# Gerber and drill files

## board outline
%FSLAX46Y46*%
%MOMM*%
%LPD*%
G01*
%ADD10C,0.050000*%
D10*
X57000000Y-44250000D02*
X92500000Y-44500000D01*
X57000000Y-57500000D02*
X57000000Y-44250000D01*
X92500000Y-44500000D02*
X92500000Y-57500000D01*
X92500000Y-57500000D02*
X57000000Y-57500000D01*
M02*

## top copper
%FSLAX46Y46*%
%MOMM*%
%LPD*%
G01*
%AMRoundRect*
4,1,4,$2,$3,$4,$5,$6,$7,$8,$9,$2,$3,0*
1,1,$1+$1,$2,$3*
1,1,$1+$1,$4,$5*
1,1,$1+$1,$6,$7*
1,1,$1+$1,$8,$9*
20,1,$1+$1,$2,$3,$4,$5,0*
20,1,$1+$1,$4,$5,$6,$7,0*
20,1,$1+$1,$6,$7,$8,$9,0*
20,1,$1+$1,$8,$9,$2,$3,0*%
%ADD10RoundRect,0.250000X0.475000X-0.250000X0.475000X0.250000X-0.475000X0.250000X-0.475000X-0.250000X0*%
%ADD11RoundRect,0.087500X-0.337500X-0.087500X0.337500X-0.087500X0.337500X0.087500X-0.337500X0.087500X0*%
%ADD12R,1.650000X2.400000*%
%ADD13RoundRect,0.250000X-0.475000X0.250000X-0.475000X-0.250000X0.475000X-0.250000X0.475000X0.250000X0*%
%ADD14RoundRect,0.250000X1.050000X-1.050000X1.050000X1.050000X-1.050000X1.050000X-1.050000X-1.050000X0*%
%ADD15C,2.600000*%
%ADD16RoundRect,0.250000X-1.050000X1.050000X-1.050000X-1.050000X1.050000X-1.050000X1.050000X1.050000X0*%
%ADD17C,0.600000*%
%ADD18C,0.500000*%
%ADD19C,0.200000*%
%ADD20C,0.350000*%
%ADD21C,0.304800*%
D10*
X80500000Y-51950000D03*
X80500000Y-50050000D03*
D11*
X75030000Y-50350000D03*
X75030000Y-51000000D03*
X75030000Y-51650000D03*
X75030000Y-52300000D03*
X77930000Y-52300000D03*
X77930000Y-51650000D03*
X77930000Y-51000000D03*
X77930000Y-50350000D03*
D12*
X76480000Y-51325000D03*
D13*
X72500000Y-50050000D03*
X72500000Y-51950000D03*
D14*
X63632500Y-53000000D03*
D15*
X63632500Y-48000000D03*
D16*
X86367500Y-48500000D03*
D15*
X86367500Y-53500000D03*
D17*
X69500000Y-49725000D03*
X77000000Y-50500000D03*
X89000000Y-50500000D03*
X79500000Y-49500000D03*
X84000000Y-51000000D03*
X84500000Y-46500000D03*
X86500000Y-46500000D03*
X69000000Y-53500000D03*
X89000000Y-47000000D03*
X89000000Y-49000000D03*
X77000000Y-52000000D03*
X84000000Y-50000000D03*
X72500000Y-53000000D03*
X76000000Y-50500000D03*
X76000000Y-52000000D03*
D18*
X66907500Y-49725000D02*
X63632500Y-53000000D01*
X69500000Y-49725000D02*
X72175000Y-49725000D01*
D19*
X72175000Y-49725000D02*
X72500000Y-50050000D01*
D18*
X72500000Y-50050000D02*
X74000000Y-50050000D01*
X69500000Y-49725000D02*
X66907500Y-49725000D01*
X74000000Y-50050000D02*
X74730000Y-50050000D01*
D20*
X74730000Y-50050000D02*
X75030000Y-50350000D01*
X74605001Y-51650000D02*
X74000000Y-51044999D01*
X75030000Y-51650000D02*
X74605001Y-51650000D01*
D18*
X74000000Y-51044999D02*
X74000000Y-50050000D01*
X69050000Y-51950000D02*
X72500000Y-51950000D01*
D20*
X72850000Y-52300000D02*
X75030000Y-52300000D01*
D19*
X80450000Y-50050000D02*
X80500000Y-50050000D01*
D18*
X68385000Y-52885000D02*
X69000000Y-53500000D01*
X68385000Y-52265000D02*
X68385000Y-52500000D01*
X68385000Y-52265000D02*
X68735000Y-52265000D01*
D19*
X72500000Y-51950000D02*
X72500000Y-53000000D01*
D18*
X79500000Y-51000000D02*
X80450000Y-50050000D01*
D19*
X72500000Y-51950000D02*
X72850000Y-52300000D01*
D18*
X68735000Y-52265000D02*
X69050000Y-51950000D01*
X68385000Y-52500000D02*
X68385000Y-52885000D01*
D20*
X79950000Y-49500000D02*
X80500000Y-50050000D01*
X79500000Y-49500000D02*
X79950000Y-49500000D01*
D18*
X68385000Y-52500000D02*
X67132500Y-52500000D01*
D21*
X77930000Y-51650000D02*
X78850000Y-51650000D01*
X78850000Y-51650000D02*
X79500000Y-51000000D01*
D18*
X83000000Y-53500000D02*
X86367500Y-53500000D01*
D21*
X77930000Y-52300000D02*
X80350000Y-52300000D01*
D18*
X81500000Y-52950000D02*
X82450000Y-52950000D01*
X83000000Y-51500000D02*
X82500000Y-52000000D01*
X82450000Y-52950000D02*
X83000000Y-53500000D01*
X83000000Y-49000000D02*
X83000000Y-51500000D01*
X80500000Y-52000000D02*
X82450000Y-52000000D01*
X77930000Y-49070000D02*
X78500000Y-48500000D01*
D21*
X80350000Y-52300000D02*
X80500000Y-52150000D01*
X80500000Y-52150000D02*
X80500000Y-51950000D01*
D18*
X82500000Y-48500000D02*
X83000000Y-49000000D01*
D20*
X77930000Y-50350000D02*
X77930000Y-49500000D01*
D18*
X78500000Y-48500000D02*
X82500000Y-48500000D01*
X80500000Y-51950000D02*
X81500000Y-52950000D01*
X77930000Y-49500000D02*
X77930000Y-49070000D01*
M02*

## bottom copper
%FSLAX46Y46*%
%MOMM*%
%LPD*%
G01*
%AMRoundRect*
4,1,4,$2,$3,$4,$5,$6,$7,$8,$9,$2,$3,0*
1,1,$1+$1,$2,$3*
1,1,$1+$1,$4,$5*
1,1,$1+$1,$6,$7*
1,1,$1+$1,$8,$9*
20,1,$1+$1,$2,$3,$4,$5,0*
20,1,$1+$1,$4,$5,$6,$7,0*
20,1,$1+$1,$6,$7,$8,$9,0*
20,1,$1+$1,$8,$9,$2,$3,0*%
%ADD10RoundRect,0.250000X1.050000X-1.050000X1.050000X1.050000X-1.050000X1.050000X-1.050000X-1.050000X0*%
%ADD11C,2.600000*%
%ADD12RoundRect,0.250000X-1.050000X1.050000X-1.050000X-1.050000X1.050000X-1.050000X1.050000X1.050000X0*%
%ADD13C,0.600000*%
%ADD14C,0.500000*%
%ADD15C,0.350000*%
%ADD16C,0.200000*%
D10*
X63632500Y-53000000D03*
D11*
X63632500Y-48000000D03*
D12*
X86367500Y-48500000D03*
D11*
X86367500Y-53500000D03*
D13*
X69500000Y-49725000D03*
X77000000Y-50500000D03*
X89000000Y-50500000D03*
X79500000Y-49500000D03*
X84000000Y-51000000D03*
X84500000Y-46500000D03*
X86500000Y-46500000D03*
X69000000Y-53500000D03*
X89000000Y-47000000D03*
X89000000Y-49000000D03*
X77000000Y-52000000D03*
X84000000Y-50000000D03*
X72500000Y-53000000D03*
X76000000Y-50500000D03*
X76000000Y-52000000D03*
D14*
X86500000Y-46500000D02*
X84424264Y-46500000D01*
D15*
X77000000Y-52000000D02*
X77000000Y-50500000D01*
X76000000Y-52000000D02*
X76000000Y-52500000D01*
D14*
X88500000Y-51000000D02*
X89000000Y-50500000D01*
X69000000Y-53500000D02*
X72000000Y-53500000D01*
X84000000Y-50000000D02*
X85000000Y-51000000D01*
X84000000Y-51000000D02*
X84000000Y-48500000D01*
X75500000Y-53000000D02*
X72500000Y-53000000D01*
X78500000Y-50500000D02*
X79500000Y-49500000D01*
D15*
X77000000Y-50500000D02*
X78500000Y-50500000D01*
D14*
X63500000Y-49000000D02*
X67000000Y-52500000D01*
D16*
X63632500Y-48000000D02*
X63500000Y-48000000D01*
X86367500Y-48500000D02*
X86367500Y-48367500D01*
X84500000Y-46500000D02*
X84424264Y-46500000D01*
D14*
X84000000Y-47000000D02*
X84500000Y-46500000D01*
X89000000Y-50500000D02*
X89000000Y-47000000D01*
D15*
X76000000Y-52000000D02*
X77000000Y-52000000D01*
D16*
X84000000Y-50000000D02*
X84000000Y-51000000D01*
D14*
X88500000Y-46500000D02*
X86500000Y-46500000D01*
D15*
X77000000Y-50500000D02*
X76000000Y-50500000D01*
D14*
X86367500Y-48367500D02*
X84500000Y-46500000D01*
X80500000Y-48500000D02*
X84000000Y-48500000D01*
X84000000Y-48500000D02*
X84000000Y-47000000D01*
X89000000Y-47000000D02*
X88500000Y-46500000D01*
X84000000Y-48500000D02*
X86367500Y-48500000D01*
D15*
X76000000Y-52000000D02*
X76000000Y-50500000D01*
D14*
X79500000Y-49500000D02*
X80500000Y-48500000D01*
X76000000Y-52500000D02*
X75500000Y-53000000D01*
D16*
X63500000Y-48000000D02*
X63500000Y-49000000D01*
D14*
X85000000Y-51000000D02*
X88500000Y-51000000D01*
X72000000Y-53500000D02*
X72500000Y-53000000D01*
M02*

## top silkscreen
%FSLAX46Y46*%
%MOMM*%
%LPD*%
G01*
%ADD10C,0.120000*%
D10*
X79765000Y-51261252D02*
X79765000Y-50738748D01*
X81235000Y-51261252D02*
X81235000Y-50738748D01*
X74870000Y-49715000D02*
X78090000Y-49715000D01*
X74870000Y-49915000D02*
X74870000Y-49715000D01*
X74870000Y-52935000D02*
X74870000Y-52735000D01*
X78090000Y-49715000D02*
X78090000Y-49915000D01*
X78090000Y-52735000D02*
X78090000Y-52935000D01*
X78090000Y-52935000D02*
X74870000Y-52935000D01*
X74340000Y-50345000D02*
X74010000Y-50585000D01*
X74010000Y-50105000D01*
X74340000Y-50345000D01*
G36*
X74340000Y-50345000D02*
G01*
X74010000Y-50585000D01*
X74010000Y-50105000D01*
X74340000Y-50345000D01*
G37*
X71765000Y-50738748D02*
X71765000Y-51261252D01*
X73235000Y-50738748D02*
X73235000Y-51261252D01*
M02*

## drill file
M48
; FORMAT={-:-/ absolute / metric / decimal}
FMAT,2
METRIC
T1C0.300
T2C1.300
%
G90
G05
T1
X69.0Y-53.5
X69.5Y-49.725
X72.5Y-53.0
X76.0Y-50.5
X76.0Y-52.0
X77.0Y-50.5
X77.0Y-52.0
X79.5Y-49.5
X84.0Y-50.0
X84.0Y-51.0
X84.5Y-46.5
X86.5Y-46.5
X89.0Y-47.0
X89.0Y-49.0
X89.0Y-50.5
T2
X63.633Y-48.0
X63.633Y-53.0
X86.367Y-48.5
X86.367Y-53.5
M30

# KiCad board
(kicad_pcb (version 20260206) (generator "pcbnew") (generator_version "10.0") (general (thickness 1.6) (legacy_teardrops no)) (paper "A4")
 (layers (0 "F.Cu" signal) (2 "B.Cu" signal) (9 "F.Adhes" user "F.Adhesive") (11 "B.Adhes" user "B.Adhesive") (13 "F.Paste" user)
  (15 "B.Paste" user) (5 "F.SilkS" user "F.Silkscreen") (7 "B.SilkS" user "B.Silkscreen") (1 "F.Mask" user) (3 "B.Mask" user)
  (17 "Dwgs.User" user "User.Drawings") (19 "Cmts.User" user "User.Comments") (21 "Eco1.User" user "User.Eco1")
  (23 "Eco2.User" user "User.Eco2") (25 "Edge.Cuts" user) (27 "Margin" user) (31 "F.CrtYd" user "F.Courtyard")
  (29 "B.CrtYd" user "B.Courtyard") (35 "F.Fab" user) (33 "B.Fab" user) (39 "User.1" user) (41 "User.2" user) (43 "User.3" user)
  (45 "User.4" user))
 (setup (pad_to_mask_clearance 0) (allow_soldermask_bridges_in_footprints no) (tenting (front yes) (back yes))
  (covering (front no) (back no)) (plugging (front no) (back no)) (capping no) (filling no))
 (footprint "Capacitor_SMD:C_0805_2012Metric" (layer "F.Cu") (at 80.5 51 90)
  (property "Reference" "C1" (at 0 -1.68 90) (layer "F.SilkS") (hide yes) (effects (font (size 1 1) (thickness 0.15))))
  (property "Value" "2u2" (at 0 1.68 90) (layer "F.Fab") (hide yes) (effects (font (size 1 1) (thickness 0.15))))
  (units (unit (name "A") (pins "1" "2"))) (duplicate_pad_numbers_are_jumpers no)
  (fp_line (start -0.261252 -0.735) (end 0.261252 -0.735) (stroke (width 0.12) (type solid)) (layer "F.SilkS"))
  (fp_line (start -0.261252 0.735) (end 0.261252 0.735) (stroke (width 0.12) (type solid)) (layer "F.SilkS"))
  (pad "1" smd roundrect (at -0.95 0 90) (size 1 1.45) (layers "F.Cu" "F.Mask" "F.Paste") (roundrect_rratio 0.25) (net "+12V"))
  (pad "2" smd roundrect (at 0.95 0 90) (size 1 1.45) (layers "F.Cu" "F.Mask" "F.Paste") (roundrect_rratio 0.25) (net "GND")))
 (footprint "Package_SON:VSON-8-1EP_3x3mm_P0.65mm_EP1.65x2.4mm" (layer "F.Cu") (at 76.48 51.325)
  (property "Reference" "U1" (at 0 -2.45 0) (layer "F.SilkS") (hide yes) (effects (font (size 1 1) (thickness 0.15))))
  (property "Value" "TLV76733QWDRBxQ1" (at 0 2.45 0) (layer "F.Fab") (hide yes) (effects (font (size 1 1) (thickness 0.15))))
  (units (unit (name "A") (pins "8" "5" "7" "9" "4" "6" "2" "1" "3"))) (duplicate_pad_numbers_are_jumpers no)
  (fp_line (start -1.61 -1.61) (end 1.61 -1.61) (stroke (width 0.12) (type solid)) (layer "F.SilkS"))
  (fp_line (start -1.61 -1.41) (end -1.61 -1.61) (stroke (width 0.12) (type solid)) (layer "F.SilkS"))
  (fp_line (start -1.61 1.61) (end -1.61 1.41) (stroke (width 0.12) (type solid)) (layer "F.SilkS"))
  (fp_line (start 1.61 -1.61) (end 1.61 -1.41) (stroke (width 0.12) (type solid)) (layer "F.SilkS"))
  (fp_line (start 1.61 1.41) (end 1.61 1.61) (stroke (width 0.12) (type solid)) (layer "F.SilkS"))
  (fp_line (start 1.61 1.61) (end -1.61 1.61) (stroke (width 0.12) (type solid)) (layer "F.SilkS"))
  (fp_poly (pts (xy -2.14 -0.98) (xy -2.47 -0.74) (xy -2.47 -1.22)) (stroke (width 0.12) (type solid)) (fill yes) (layer "F.SilkS"))
  (pad "" smd roundrect (at 0 -0.6) (size 1.33 0.97) (layers "F.Paste") (roundrect_rratio 0.25))
  (pad "" smd roundrect (at 0 0.6) (size 1.33 0.97) (layers "F.Paste") (roundrect_rratio 0.25))
  (pad "1" smd roundrect (at -1.45 -0.975) (size 0.85 0.35) (layers "F.Cu" "F.Mask" "F.Paste") (roundrect_rratio 0.25) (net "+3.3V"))
  (pad "2" smd roundrect (at -1.45 -0.325) (size 0.85 0.35) (layers "F.Cu" "F.Mask" "F.Paste") (roundrect_rratio 0.25)
   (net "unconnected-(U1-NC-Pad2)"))
  (pad "3" smd roundrect (at -1.45 0.325) (size 0.85 0.35) (layers "F.Cu" "F.Mask" "F.Paste") (roundrect_rratio 0.25) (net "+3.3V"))
  (pad "4" smd roundrect (at -1.45 0.975) (size 0.85 0.35) (layers "F.Cu" "F.Mask" "F.Paste") (roundrect_rratio 0.25) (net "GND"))
  (pad "5" smd roundrect (at 1.45 0.975) (size 0.85 0.35) (layers "F.Cu" "F.Mask" "F.Paste") (roundrect_rratio 0.25) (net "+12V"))
  (pad "6" smd roundrect (at 1.45 0.325) (size 0.85 0.35) (layers "F.Cu" "F.Mask" "F.Paste") (roundrect_rratio 0.25) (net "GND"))
  (pad "7" smd roundrect (at 1.45 -0.325) (size 0.85 0.35) (layers "F.Cu" "F.Mask" "F.Paste") (roundrect_rratio 0.25)
   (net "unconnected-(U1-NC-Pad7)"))
  (pad "8" smd roundrect (at 1.45 -0.975) (size 0.85 0.35) (layers "F.Cu" "F.Mask" "F.Paste") (roundrect_rratio 0.25) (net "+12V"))
  (pad "9" smd rect (at 0 0) (size 1.65 2.4) (layers "F.Cu" "F.Mask") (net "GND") (zone_connect 2)))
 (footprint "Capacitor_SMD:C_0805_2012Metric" (layer "F.Cu") (at 72.5 51 -90)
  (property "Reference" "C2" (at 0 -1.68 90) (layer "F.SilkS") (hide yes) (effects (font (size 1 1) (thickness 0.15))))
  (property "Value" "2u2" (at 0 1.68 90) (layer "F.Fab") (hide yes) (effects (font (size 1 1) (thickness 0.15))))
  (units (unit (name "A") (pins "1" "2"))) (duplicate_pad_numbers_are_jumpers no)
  (fp_line (start -0.261252 0.735) (end 0.261252 0.735) (stroke (width 0.12) (type solid)) (layer "F.SilkS"))
  (fp_line (start -0.261252 -0.735) (end 0.261252 -0.735) (stroke (width 0.12) (type solid)) (layer "F.SilkS"))
  (pad "1" smd roundrect (at -0.95 0 270) (size 1 1.45) (layers "F.Cu" "F.Mask" "F.Paste") (roundrect_rratio 0.25) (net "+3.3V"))
  (pad "2" smd roundrect (at 0.95 0 270) (size 1 1.45) (layers "F.Cu" "F.Mask" "F.Paste") (roundrect_rratio 0.25) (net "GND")))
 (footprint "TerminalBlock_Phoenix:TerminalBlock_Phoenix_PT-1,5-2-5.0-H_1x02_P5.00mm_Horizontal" (layer "B.Cu") (at 63.6325 53 90)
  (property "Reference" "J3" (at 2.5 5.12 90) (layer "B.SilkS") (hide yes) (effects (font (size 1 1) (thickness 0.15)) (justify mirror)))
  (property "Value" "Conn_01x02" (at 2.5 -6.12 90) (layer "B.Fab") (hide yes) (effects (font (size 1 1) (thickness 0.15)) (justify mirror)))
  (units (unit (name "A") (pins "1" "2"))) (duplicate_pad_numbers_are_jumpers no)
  (pad "1" thru_hole roundrect (at 0 0 90) (size 2.6 2.6) (drill 1.3) (layers "*.Cu" "*.Mask") (remove_unused_layers no)
   (roundrect_rratio 0.096154) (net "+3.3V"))
  (pad "2" thru_hole circle (at 5 0 90) (size 2.6 2.6) (drill 1.3) (layers "*.Cu" "*.Mask") (remove_unused_layers no) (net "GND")))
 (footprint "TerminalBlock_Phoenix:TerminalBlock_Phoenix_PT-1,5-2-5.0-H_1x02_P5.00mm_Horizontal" (layer "B.Cu") (at 86.3675 48.5 -90)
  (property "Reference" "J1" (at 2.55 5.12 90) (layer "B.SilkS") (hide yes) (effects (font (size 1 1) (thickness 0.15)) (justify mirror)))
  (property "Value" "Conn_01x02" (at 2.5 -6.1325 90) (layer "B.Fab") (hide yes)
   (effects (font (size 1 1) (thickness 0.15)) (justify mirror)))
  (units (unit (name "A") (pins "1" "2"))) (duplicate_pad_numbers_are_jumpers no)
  (pad "1" thru_hole roundrect (at 0 0 270) (size 2.6 2.6) (drill 1.3) (layers "*.Cu" "*.Mask") (remove_unused_layers no)
   (roundrect_rratio 0.096154) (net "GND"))
  (pad "2" thru_hole circle (at 5 0 270) (size 2.6 2.6) (drill 1.3) (layers "*.Cu" "*.Mask") (remove_unused_layers no) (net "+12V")))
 (gr_line (start 57 44.25) (end 92.5 44.5) (stroke (width 0.05) (type default)) (layer "Edge.Cuts"))
 (gr_line (start 57 57.5) (end 57 44.25) (stroke (width 0.05) (type default)) (layer "Edge.Cuts"))
 (gr_line (start 92.5 44.5) (end 92.5 57.5) (stroke (width 0.05) (type default)) (layer "Edge.Cuts"))
 (gr_line (start 92.5 57.5) (end 57 57.5) (stroke (width 0.05) (type solid)) (layer "Edge.Cuts"))
 (segment (start 66.9075 49.725) (end 63.6325 53) (width 0.5) (layer "F.Cu") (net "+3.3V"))
 (segment (start 69.5 49.725) (end 72.175 49.725) (width 0.5) (layer "F.Cu") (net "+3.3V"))
 (segment (start 72.175 49.725) (end 72.5 50.05) (width 0.2) (layer "F.Cu") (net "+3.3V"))
 (segment (start 72.5 50.05) (end 74 50.05) (width 0.5) (layer "F.Cu") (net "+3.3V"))
 (segment (start 69.5 49.725) (end 66.9075 49.725) (width 0.5) (layer "F.Cu") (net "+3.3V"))
 (segment (start 74 50.05) (end 74.73 50.05) (width 0.5) (layer "F.Cu") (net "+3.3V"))
 (segment (start 74.73 50.05) (end 75.03 50.35) (width 0.35) (layer "F.Cu") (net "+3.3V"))
 (segment (start 74.605001 51.65) (end 74 51.044999) (width 0.35) (layer "F.Cu") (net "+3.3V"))
 (segment (start 75.03 51.65) (end 74.605001 51.65) (width 0.35) (layer "F.Cu") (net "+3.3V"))
 (segment (start 74 51.044999) (end 74 50.05) (width 0.5) (layer "F.Cu") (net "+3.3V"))
 (via (at 69.5 49.725) (size 0.6) (drill 0.3) (layers "F.Cu" "B.Cu") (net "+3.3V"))
 (segment (start 69.05 51.95) (end 72.5 51.95) (width 0.5) (layer "F.Cu") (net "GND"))
 (segment (start 72.85 52.3) (end 75.03 52.3) (width 0.35) (layer "F.Cu") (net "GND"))
 (segment (start 80.45 50.05) (end 80.5 50.05) (width 0.2) (layer "F.Cu") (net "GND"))
 (segment (start 68.385 52.885) (end 69 53.5) (width 0.5) (layer "F.Cu") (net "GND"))
 (segment (start 68.385 52.265) (end 68.385 52.5) (width 0.5) (layer "F.Cu") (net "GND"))
 (segment (start 68.385 52.265) (end 68.735 52.265) (width 0.5) (layer "F.Cu") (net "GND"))
 (segment (start 72.5 51.95) (end 72.5 53) (width 0.2) (layer "F.Cu") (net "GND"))
 (segment (start 79.5 51) (end 80.45 50.05) (width 0.5) (layer "F.Cu") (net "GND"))
 (segment (start 72.5 51.95) (end 72.85 52.3) (width 0.2) (layer "F.Cu") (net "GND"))
 (segment (start 68.735 52.265) (end 69.05 51.95) (width 0.5) (layer "F.Cu") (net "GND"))
 (segment (start 68.385 52.5) (end 68.385 52.885) (width 0.5) (layer "F.Cu") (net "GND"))
 (segment (start 79.95 49.5) (end 80.5 50.05) (width 0.35) (layer "F.Cu") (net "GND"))
 (segment (start 79.5 49.5) (end 79.95 49.5) (width 0.35) (layer "F.Cu") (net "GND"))
 (segment (start 68.385 52.5) (end 67.1325 52.5) (width 0.5) (layer "F.Cu") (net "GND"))
 (segment (start 77.93 51.65) (end 78.85 51.65) (width 0.3048) (layer "F.Cu") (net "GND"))
 (segment (start 78.85 51.65) (end 79.5 51) (width 0.3048) (layer "F.Cu") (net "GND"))
 (via (at 77 50.5) (size 0.6) (drill 0.3) (layers "F.Cu" "B.Cu") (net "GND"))
 (via (at 89 50.5) (size 0.6) (drill 0.3) (layers "F.Cu" "B.Cu") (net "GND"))
 (via (at 79.5 49.5) (size 0.6) (drill 0.3) (layers "F.Cu" "B.Cu") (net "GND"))
 (via (at 84 51) (size 0.6) (drill 0.3) (layers "F.Cu" "B.Cu") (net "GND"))
 (via (at 84.5 46.5) (size 0.6) (drill 0.3) (layers "F.Cu" "B.Cu") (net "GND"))
 (via (at 86.5 46.5) (size 0.6) (drill 0.3) (layers "F.Cu" "B.Cu") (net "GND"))
 (via (at 69 53.5) (size 0.6) (drill 0.3) (layers "F.Cu" "B.Cu") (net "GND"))
 (via (at 89 47) (size 0.6) (drill 0.3) (layers "F.Cu" "B.Cu") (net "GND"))
 (via (at 89 49) (size 0.6) (drill 0.3) (layers "F.Cu" "B.Cu") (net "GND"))
 (via (at 77 52) (size 0.6) (drill 0.3) (layers "F.Cu" "B.Cu") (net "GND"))
 (via (at 84 50) (size 0.6) (drill 0.3) (layers "F.Cu" "B.Cu") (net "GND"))
 (via (at 72.5 53) (size 0.6) (drill 0.3) (layers "F.Cu" "B.Cu") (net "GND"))
 (via (at 76 50.5) (size 0.6) (drill 0.3) (layers "F.Cu" "B.Cu") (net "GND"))
 (via (at 76 52) (size 0.6) (drill 0.3) (layers "F.Cu" "B.Cu") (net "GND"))
 (segment (start 86.5 46.5) (end 84.424264 46.5) (width 0.5) (layer "B.Cu") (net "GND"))
 (segment (start 77 52) (end 77 50.5) (width 0.35) (layer "B.Cu") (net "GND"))
 (segment (start 76 52) (end 76 52.5) (width 0.35) (layer "B.Cu") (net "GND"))
 (segment (start 88.5 51) (end 89 50.5) (width 0.5) (layer "B.Cu") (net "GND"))
 (segment (start 69 53.5) (end 72 53.5) (width 0.5) (layer "B.Cu") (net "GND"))
 (segment (start 84 50) (end 85 51) (width 0.5) (layer "B.Cu") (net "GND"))
 (segment (start 84 51) (end 84 48.5) (width 0.5) (layer "B.Cu") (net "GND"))
 (segment (start 75.5 53) (end 72.5 53) (width 0.5) (layer "B.Cu") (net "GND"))
 (segment (start 78.5 50.5) (end 79.5 49.5) (width 0.5) (layer "B.Cu") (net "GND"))
 (segment (start 77 50.5) (end 78.5 50.5) (width 0.35) (layer "B.Cu") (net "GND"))
 (segment (start 63.5 49) (end 67 52.5) (width 0.5) (layer "B.Cu") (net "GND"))
 (segment (start 63.6325 48) (end 63.5 48) (width 0.2) (layer "B.Cu") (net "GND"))
 (segment (start 86.3675 48.5) (end 86.3675 48.3675) (width 0.2) (layer "B.Cu") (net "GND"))
 (segment (start 84.5 46.5) (end 84.424264 46.5) (width 0.2) (layer "B.Cu") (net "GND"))
 (segment (start 84 47) (end 84.5 46.5) (width 0.5) (layer "B.Cu") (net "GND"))
 (segment (start 89 50.5) (end 89 47) (width 0.5) (layer "B.Cu") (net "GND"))
 (segment (start 76 52) (end 77 52) (width 0.35) (layer "B.Cu") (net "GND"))
 (segment (start 84 50) (end 84 51) (width 0.2) (layer "B.Cu") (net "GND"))
 (segment (start 88.5 46.5) (end 86.5 46.5) (width 0.5) (layer "B.Cu") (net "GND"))
 (segment (start 77 50.5) (end 76 50.5) (width 0.35) (layer "B.Cu") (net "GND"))
 (segment (start 86.3675 48.3675) (end 84.5 46.5) (width 0.5) (layer "B.Cu") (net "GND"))
 (segment (start 80.5 48.5) (end 84 48.5) (width 0.5) (layer "B.Cu") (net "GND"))
 (segment (start 84 48.5) (end 84 47) (width 0.5) (layer "B.Cu") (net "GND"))
 (segment (start 89 47) (end 88.5 46.5) (width 0.5) (layer "B.Cu") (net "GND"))
 (segment (start 84 48.5) (end 86.3675 48.5) (width 0.5) (layer "B.Cu") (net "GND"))
 (segment (start 76 52) (end 76 50.5) (width 0.35) (layer "B.Cu") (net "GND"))
 (segment (start 79.5 49.5) (end 80.5 48.5) (width 0.5) (layer "B.Cu") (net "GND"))
 (segment (start 76 52.5) (end 75.5 53) (width 0.5) (layer "B.Cu") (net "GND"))
 (segment (start 63.5 48) (end 63.5 49) (width 0.2) (layer "B.Cu") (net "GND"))
 (segment (start 85 51) (end 88.5 51) (width 0.5) (layer "B.Cu") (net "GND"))
 (segment (start 72 53.5) (end 72.5 53) (width 0.5) (layer "B.Cu") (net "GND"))
 (segment (start 83 53.5) (end 86.3675 53.5) (width 0.5) (layer "F.Cu") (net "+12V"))
 (segment (start 77.93 52.3) (end 80.35 52.3) (width 0.3048) (layer "F.Cu") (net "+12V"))
 (segment (start 81.5 52.95) (end 82.45 52.95) (width 0.5) (layer "F.Cu") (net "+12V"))
 (segment (start 83 51.5) (end 82.5 52) (width 0.5) (layer "F.Cu") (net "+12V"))
 (segment (start 82.45 52.95) (end 83 53.5) (width 0.5) (layer "F.Cu") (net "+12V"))
 (segment (start 83 49) (end 83 51.5) (width 0.5) (layer "F.Cu") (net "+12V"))
 (segment (start 80.5 52) (end 82.45 52) (width 0.5) (layer "F.Cu") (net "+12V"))
 (segment (start 77.93 49.07) (end 78.5 48.5) (width 0.5) (layer "F.Cu") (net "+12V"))
 (segment (start 80.35 52.3) (end 80.5 52.15) (width 0.3048) (layer "F.Cu") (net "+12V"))
 (segment (start 80.5 52.15) (end 80.5 51.95) (width 0.3048) (layer "F.Cu") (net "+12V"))
 (segment (start 82.5 48.5) (end 83 49) (width 0.5) (layer "F.Cu") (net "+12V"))
 (segment (start 77.93 50.35) (end 77.93 49.5) (width 0.35) (layer "F.Cu") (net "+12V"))
 (segment (start 78.5 48.5) (end 82.5 48.5) (width 0.5) (layer "F.Cu") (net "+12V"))
 (segment (start 80.5 51.95) (end 81.5 52.95) (width 0.5) (layer "F.Cu") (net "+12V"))
 (segment (start 77.93 49.5) (end 77.93 49.07) (width 0.5) (layer "F.Cu") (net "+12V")))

